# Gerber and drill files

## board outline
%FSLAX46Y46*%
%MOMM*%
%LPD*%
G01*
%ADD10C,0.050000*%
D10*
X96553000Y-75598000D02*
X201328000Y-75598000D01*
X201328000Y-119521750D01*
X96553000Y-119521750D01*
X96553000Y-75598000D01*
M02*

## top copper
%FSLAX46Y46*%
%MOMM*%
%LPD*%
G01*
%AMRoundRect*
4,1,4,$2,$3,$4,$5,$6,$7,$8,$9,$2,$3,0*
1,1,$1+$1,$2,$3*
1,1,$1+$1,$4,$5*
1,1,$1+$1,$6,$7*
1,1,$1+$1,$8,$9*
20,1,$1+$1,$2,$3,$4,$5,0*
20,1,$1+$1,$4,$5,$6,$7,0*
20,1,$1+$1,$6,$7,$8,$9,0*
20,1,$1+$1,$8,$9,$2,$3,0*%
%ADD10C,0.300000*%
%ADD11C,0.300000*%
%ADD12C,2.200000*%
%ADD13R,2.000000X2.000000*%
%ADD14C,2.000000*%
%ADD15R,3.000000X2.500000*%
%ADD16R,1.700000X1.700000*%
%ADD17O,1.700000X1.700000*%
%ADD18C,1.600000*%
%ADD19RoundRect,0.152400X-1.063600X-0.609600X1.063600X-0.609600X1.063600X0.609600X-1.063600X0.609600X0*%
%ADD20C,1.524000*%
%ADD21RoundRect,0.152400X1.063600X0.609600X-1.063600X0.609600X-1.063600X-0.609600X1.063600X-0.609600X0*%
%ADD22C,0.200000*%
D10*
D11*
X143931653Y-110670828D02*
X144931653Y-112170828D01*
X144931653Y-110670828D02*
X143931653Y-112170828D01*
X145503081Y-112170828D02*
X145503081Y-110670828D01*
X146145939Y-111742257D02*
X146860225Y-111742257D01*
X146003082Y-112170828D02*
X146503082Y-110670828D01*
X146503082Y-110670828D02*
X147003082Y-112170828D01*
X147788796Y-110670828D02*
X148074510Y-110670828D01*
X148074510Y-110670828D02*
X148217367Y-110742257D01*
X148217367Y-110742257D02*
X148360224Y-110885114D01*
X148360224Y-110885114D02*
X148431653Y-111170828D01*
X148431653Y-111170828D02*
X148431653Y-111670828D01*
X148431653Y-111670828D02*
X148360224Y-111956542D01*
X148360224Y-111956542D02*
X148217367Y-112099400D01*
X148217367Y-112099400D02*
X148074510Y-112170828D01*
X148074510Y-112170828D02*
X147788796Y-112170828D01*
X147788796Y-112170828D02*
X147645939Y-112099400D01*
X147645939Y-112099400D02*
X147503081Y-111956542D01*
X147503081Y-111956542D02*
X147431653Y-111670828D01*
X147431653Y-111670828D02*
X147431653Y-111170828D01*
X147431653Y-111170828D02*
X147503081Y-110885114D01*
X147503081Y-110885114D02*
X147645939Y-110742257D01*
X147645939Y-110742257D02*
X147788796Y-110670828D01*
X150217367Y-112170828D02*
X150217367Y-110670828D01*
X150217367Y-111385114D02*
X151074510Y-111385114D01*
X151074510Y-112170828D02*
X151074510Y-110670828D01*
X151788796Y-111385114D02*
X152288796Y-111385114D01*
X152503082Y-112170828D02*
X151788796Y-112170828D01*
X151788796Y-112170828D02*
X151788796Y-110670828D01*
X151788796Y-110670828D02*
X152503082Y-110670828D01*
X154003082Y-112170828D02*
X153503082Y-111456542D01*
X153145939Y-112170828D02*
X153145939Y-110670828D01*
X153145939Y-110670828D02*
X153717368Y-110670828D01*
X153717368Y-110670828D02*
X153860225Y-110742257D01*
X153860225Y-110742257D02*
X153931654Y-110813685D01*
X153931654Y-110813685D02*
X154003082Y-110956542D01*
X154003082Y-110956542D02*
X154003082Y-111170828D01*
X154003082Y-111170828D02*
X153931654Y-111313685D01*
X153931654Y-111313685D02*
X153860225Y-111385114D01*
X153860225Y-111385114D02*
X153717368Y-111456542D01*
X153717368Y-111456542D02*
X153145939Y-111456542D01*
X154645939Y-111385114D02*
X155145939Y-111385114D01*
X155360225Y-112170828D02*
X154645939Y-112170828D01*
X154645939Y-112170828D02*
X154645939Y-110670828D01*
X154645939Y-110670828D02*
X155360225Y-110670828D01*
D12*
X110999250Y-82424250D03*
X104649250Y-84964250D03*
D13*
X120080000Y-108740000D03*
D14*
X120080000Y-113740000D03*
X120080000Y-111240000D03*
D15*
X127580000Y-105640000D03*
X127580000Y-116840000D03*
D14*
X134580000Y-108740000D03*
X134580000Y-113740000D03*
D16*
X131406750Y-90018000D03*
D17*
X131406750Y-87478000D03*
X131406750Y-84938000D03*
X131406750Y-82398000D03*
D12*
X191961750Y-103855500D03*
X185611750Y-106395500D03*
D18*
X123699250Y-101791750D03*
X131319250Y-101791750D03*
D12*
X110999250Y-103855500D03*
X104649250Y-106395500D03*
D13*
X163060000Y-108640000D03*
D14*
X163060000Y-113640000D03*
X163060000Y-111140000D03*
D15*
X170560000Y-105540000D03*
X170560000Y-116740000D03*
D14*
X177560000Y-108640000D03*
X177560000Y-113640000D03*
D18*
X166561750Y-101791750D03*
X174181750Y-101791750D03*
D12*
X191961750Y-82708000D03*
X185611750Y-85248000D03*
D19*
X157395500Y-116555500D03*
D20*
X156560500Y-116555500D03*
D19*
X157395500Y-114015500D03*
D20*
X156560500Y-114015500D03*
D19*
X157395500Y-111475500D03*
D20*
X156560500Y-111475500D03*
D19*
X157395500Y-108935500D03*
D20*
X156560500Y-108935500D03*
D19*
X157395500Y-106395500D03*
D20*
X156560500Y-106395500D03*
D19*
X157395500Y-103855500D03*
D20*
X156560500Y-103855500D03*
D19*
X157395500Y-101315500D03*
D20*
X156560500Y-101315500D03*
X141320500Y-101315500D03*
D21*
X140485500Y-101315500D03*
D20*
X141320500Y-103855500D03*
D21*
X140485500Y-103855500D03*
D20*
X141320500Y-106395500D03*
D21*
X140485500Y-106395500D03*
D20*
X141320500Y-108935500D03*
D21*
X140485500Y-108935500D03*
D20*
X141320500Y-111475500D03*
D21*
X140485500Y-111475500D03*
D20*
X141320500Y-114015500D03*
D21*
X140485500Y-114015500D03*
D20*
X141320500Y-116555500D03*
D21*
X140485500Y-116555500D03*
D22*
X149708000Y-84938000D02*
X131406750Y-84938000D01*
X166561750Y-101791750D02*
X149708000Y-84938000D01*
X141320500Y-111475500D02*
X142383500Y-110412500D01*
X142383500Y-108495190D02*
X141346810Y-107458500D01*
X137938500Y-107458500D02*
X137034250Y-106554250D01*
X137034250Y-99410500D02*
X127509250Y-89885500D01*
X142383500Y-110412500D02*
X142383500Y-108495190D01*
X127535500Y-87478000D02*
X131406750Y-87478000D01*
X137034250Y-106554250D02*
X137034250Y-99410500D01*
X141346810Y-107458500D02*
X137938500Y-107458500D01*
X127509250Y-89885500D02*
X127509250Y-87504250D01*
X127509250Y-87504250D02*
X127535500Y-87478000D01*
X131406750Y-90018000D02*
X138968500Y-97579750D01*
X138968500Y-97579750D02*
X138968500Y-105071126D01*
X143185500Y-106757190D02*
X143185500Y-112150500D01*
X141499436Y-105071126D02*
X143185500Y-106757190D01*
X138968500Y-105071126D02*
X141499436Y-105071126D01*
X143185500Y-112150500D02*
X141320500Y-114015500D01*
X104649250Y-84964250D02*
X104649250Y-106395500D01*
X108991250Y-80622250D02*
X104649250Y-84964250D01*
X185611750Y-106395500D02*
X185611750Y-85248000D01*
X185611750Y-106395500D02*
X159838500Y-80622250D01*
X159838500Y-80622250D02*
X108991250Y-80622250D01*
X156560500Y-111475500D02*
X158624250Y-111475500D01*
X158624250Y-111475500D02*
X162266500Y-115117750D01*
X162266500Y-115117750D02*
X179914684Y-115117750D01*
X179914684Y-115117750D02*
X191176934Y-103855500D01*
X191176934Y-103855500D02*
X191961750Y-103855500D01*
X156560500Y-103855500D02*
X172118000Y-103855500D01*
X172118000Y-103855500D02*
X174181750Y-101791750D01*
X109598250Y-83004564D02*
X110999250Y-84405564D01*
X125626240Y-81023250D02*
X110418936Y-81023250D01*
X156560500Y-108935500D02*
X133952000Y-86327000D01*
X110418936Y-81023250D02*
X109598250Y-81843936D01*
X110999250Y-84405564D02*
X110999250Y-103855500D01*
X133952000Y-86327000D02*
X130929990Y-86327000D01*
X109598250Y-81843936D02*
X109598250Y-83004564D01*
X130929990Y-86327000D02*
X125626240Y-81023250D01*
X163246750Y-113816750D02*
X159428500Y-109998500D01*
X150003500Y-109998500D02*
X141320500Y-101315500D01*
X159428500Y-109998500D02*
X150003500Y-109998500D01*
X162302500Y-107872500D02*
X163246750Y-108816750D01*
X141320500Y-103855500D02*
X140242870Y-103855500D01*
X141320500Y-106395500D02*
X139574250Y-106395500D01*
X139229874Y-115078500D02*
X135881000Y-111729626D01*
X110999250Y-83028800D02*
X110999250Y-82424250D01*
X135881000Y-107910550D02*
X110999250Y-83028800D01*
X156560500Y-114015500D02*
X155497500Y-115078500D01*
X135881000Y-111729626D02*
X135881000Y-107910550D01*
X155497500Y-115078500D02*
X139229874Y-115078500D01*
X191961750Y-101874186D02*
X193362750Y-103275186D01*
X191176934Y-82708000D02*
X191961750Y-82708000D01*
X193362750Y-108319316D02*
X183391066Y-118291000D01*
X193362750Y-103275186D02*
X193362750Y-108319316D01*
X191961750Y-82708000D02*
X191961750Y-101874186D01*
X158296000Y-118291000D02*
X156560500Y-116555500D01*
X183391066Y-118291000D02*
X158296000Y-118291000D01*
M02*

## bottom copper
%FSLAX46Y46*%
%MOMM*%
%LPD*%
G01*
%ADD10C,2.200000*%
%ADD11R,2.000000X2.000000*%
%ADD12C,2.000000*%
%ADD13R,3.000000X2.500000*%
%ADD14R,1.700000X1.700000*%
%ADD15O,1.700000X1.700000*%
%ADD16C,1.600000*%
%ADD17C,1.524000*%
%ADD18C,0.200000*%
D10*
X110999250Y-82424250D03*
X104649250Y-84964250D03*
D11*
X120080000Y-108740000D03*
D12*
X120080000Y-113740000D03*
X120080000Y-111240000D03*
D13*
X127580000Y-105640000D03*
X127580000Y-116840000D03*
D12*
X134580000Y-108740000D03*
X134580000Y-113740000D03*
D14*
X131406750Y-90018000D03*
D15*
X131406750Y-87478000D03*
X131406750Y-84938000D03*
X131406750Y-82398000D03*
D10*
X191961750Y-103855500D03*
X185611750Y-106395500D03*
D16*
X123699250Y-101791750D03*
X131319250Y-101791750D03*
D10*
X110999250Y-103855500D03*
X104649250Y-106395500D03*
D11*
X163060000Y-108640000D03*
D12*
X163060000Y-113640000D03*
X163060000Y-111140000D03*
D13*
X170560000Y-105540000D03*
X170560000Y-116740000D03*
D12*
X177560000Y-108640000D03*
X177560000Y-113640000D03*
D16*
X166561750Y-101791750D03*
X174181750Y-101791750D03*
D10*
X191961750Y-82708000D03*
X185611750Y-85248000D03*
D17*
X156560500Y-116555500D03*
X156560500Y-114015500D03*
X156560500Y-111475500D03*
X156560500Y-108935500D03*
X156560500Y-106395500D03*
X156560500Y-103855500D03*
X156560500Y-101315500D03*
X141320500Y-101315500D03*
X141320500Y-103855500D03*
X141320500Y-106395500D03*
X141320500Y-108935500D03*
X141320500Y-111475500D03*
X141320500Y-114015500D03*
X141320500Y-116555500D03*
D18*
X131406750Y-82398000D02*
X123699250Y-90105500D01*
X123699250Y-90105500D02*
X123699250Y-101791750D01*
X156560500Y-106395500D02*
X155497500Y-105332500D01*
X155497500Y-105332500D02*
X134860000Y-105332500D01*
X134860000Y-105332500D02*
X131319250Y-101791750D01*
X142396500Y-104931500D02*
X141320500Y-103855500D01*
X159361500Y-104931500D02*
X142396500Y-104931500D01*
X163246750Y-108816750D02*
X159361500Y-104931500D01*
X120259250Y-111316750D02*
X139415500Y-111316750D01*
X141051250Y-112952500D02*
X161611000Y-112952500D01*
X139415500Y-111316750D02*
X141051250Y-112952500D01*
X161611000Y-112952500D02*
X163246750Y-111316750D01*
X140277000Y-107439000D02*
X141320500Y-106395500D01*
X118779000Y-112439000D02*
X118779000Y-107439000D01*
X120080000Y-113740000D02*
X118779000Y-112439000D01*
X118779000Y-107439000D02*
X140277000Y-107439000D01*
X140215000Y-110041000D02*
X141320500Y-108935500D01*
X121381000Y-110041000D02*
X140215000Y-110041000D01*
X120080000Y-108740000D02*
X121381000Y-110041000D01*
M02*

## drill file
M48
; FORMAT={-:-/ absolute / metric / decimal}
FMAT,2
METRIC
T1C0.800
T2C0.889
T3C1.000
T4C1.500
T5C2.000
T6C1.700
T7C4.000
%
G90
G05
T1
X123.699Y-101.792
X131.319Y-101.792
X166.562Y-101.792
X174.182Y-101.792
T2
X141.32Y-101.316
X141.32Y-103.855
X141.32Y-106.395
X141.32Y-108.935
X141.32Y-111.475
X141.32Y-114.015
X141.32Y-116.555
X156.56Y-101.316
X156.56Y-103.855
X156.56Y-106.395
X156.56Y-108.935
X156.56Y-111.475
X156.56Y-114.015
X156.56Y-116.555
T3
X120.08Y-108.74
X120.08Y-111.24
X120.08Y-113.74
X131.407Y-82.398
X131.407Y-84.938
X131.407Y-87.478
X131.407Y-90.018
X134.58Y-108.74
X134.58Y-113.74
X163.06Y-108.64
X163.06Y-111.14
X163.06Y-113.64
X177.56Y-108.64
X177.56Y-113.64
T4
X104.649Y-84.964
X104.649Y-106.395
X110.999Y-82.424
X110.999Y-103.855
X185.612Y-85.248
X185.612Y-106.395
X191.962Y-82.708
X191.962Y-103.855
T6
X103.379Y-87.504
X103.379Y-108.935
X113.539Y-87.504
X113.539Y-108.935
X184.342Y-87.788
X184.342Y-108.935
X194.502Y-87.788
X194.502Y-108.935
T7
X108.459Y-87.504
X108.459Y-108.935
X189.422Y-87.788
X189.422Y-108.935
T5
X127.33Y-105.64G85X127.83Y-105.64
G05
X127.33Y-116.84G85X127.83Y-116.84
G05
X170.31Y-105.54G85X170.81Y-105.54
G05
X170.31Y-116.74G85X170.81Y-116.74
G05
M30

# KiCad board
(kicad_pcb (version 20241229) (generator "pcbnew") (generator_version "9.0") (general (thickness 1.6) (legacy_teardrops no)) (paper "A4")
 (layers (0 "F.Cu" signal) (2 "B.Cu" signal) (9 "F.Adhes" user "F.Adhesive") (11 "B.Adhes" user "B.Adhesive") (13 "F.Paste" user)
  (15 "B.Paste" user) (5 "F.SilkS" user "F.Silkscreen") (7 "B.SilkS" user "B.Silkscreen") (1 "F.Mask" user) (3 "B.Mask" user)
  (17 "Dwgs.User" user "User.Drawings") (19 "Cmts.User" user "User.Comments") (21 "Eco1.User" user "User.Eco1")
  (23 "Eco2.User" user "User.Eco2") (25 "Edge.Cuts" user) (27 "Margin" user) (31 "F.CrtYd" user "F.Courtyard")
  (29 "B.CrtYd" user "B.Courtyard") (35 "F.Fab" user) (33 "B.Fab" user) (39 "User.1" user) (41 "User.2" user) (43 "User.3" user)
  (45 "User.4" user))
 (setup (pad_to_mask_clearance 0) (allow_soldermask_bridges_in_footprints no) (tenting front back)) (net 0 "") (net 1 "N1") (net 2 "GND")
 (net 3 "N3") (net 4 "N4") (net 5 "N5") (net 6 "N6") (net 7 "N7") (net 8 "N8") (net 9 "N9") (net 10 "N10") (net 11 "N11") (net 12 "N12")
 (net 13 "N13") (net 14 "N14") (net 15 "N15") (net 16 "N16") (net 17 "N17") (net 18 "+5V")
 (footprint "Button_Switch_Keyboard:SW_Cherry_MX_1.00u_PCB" (layer "F.Cu") (at 110.99925 82.42425)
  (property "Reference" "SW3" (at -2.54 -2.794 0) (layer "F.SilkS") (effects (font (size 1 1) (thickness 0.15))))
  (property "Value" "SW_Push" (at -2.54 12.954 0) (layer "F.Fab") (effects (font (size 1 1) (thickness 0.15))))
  (pad "" np_thru_hole circle (at -7.62 5.08) (size 1.7 1.7) (drill 1.7) (layers "*.Cu" "*.Mask"))
  (pad "" np_thru_hole circle (at -2.54 5.08) (size 4 4) (drill 4) (layers "*.Cu" "*.Mask"))
  (pad "" np_thru_hole circle (at 2.54 5.08) (size 1.7 1.7) (drill 1.7) (layers "*.Cu" "*.Mask"))
  (pad "1" thru_hole circle (at 0 0) (size 2.2 2.2) (drill 1.5) (layers "*.Cu" "*.Mask") (remove_unused_layers no) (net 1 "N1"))
  (pad "2" thru_hole circle (at -6.35 2.54) (size 2.2 2.2) (drill 1.5) (layers "*.Cu" "*.Mask") (remove_unused_layers no) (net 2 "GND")))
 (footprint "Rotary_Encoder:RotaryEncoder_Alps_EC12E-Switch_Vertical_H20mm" (layer "F.Cu") (at 120.08 108.74)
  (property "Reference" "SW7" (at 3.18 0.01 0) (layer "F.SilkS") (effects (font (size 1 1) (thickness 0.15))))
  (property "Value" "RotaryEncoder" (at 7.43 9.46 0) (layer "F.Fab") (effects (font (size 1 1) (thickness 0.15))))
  (pad "A" thru_hole rect (at 0 0) (size 2 2) (drill 1) (layers "*.Cu" "*.Mask") (remove_unused_layers no) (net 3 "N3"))
  (pad "B" thru_hole circle (at 0 5) (size 2 2) (drill 1) (layers "*.Cu" "*.Mask") (remove_unused_layers no) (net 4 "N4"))
  (pad "C" thru_hole circle (at 0 2.5) (size 2 2) (drill 1) (layers "*.Cu" "*.Mask") (remove_unused_layers no) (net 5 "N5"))
  (pad "MP" thru_hole rect (at 7.5 -3.1) (size 3 2.5) (drill oval 2.5 2) (layers "*.Cu" "*.Mask") (remove_unused_layers no))
  (pad "MP" thru_hole rect (at 7.5 8.1) (size 3 2.5) (drill oval 2.5 2) (layers "*.Cu" "*.Mask") (remove_unused_layers no))
  (pad "S1" thru_hole circle (at 14.5 0) (size 2 2) (drill 1) (layers "*.Cu" "*.Mask") (remove_unused_layers no))
  (pad "S2" thru_hole circle (at 14.5 5) (size 2 2) (drill 1) (layers "*.Cu" "*.Mask") (remove_unused_layers no)))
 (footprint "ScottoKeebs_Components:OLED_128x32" (layer "F.Cu") (at 129.80675 80.218)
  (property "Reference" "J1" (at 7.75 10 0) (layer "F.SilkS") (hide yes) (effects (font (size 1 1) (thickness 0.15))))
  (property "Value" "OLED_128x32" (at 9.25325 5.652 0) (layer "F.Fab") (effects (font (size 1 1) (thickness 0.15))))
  (pad "1" thru_hole rect (at 1.6 9.8 180) (size 1.7 1.7) (drill 1) (layers "*.Cu" "*.Mask") (remove_unused_layers no) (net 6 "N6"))
  (pad "2" thru_hole oval (at 1.6 7.26 180) (size 1.7 1.7) (drill 1) (layers "*.Cu" "*.Mask") (remove_unused_layers no) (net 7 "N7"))
  (pad "3" thru_hole oval (at 1.6 4.72 180) (size 1.7 1.7) (drill 1) (layers "*.Cu" "*.Mask") (remove_unused_layers no) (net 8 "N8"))
  (pad "4" thru_hole oval (at 1.6 2.18 180) (size 1.7 1.7) (drill 1) (layers "*.Cu" "*.Mask") (remove_unused_layers no) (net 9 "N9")))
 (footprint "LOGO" (layer "F.Cu") (at 148.86 95.36)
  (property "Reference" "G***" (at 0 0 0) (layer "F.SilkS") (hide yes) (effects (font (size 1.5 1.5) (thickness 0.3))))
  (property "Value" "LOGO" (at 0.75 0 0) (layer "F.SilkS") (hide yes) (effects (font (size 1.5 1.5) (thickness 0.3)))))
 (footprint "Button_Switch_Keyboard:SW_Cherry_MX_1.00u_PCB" (layer "F.Cu") (at 191.96175 103.8555)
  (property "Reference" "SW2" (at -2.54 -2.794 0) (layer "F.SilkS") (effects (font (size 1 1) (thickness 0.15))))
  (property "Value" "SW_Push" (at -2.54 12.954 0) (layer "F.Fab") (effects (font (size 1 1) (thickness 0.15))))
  (pad "" np_thru_hole circle (at -7.62 5.08) (size 1.7 1.7) (drill 1.7) (layers "*.Cu" "*.Mask"))
  (pad "" np_thru_hole circle (at -2.54 5.08) (size 4 4) (drill 4) (layers "*.Cu" "*.Mask"))
  (pad "" np_thru_hole circle (at 2.54 5.08) (size 1.7 1.7) (drill 1.7) (layers "*.Cu" "*.Mask"))
  (pad "1" thru_hole circle (at 0 0) (size 2.2 2.2) (drill 1.5) (layers "*.Cu" "*.Mask") (remove_unused_layers no) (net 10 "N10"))
  (pad "2" thru_hole circle (at -6.35 2.54) (size 2.2 2.2) (drill 1.5) (layers "*.Cu" "*.Mask") (remove_unused_layers no) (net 2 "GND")))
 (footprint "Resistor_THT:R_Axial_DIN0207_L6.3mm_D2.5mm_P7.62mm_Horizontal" (layer "F.Cu") (at 123.69925 101.79175)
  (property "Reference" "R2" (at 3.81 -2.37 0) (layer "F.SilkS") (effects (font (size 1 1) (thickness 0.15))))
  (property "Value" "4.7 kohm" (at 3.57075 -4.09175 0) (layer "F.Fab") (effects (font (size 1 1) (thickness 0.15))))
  (pad "1" thru_hole circle (at 0 0) (size 1.6 1.6) (drill 0.8) (layers "*.Cu" "*.Mask") (remove_unused_layers no) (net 9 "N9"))
  (pad "2" thru_hole circle (at 7.62 0) (size 1.6 1.6) (drill 0.8) (layers "*.Cu" "*.Mask") (remove_unused_layers no) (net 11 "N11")))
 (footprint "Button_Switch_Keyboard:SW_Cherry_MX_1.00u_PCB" (layer "F.Cu") (at 110.99925 103.8555)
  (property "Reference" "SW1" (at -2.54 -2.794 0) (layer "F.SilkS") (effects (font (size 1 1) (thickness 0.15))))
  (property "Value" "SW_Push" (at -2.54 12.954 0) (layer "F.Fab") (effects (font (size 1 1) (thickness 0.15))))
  (pad "" np_thru_hole circle (at -7.62 5.08) (size 1.7 1.7) (drill 1.7) (layers "*.Cu" "*.Mask"))
  (pad "" np_thru_hole circle (at -2.54 5.08) (size 4 4) (drill 4) (layers "*.Cu" "*.Mask"))
  (pad "" np_thru_hole circle (at 2.54 5.08) (size 1.7 1.7) (drill 1.7) (layers "*.Cu" "*.Mask"))
  (pad "1" thru_hole circle (at 0 0) (size 2.2 2.2) (drill 1.5) (layers "*.Cu" "*.Mask") (remove_unused_layers no) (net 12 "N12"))
  (pad "2" thru_hole circle (at -6.35 2.54) (size 2.2 2.2) (drill 1.5) (layers "*.Cu" "*.Mask") (remove_unused_layers no) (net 2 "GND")))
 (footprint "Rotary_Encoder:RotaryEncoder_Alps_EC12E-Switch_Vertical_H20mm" (layer "F.Cu") (at 163.06 108.64)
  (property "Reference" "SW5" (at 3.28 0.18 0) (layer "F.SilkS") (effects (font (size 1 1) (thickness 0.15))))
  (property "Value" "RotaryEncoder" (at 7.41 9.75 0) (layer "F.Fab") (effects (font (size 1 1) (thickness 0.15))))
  (pad "A" thru_hole rect (at 0 0) (size 2 2) (drill 1) (layers "*.Cu" "*.Mask") (remove_unused_layers no) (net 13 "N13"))
  (pad "B" thru_hole circle (at 0 5) (size 2 2) (drill 1) (layers "*.Cu" "*.Mask") (remove_unused_layers no) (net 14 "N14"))
  (pad "C" thru_hole circle (at 0 2.5) (size 2 2) (drill 1) (layers "*.Cu" "*.Mask") (remove_unused_layers no) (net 5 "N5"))
  (pad "MP" thru_hole rect (at 7.5 -3.1) (size 3 2.5) (drill oval 2.5 2) (layers "*.Cu" "*.Mask") (remove_unused_layers no))
  (pad "MP" thru_hole rect (at 7.5 8.1) (size 3 2.5) (drill oval 2.5 2) (layers "*.Cu" "*.Mask") (remove_unused_layers no))
  (pad "S1" thru_hole circle (at 14.5 0) (size 2 2) (drill 1) (layers "*.Cu" "*.Mask") (remove_unused_layers no))
  (pad "S2" thru_hole circle (at 14.5 5) (size 2 2) (drill 1) (layers "*.Cu" "*.Mask") (remove_unused_layers no)))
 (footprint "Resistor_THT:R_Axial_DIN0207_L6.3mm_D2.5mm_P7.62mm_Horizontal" (layer "F.Cu") (at 166.56175 101.79175)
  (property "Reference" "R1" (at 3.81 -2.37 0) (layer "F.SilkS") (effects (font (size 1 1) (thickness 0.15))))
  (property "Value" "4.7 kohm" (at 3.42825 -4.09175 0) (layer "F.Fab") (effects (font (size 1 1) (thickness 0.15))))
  (pad "1" thru_hole circle (at 0 0) (size 1.6 1.6) (drill 0.8) (layers "*.Cu" "*.Mask") (remove_unused_layers no) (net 8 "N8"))
  (pad "2" thru_hole circle (at 7.62 0) (size 1.6 1.6) (drill 0.8) (layers "*.Cu" "*.Mask") (remove_unused_layers no) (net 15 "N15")))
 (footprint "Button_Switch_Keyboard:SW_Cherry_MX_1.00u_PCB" (layer "F.Cu") (at 191.96175 82.708)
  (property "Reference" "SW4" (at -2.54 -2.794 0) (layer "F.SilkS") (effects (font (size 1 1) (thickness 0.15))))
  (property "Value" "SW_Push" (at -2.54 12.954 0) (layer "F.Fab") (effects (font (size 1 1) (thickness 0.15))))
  (pad "" np_thru_hole circle (at -7.62 5.08) (size 1.7 1.7) (drill 1.7) (layers "*.Cu" "*.Mask"))
  (pad "" np_thru_hole circle (at -2.54 5.08) (size 4 4) (drill 4) (layers "*.Cu" "*.Mask"))
  (pad "" np_thru_hole circle (at 2.54 5.08) (size 1.7 1.7) (drill 1.7) (layers "*.Cu" "*.Mask"))
  (pad "1" thru_hole circle (at 0 0) (size 2.2 2.2) (drill 1.5) (layers "*.Cu" "*.Mask") (remove_unused_layers no) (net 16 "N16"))
  (pad "2" thru_hole circle (at -6.35 2.54) (size 2.2 2.2) (drill 1.5) (layers "*.Cu" "*.Mask") (remove_unused_layers no) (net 2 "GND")))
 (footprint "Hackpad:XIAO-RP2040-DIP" (layer "F.Cu") (at 148.9405 108.9355 180)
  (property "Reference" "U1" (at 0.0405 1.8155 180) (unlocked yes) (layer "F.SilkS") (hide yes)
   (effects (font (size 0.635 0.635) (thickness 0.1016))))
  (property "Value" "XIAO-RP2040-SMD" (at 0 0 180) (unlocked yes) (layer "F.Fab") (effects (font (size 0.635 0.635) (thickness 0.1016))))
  (pad "1" smd roundrect (at -8.455 -7.62) (size 2.432 1.524) (layers "F.Cu" "F.Mask") (roundrect_rratio 0.1) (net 16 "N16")
   (thermal_bridge_angle 45))
  (pad "1" thru_hole circle (at -7.62 -7.62) (size 1.524 1.524) (drill 0.889) (layers "*.Cu" "*.Mask") (remove_unused_layers no)
   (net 16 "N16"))
  (pad "2" smd roundrect (at -8.455 -5.08) (size 2.432 1.524) (layers "F.Cu" "F.Mask") (roundrect_rratio 0.1) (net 1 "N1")
   (thermal_bridge_angle 45))
  (pad "2" thru_hole circle (at -7.62 -5.08) (size 1.524 1.524) (drill 0.889) (layers "*.Cu" "*.Mask") (remove_unused_layers no)
   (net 1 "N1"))
  (pad "3" smd roundrect (at -8.455 -2.54) (size 2.432 1.524) (layers "F.Cu" "F.Mask") (roundrect_rratio 0.1) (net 10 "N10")
   (thermal_bridge_angle 45))
  (pad "3" thru_hole circle (at -7.62 -2.54) (size 1.524 1.524) (drill 0.889) (layers "*.Cu" "*.Mask") (remove_unused_layers no)
   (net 10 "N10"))
  (pad "4" smd roundrect (at -8.455 0) (size 2.432 1.524) (layers "F.Cu" "F.Mask") (roundrect_rratio 0.1) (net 12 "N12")
   (thermal_bridge_angle 45))
  (pad "4" thru_hole circle (at -7.62 0) (size 1.524 1.524) (drill 0.889) (layers "*.Cu" "*.Mask") (remove_unused_layers no) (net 12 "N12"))
  (pad "5" smd roundrect (at -8.455 2.54) (size 2.432 1.524) (layers "F.Cu" "F.Mask") (roundrect_rratio 0.1) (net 11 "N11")
   (thermal_bridge_angle 45))
  (pad "5" thru_hole circle (at -7.62 2.54) (size 1.524 1.524) (drill 0.889) (layers "*.Cu" "*.Mask") (remove_unused_layers no)
   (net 11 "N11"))
  (pad "6" smd roundrect (at -8.455 5.08) (size 2.432 1.524) (layers "F.Cu" "F.Mask") (roundrect_rratio 0.1) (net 15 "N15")
   (thermal_bridge_angle 45))
  (pad "6" thru_hole circle (at -7.62 5.08) (size 1.524 1.524) (drill 0.889) (layers "*.Cu" "*.Mask") (remove_unused_layers no)
   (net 15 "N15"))
  (pad "7" smd roundrect (at -8.455 7.62) (size 2.432 1.524) (layers "F.Cu" "F.Mask") (roundrect_rratio 0.1) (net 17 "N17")
   (thermal_bridge_angle 45))
  (pad "7" thru_hole circle (at -7.62 7.62) (size 1.524 1.524) (drill 0.889) (layers "*.Cu" "*.Mask") (remove_unused_layers no)
   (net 17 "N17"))
  (pad "8" thru_hole circle (at 7.62 7.62 180) (size 1.524 1.524) (drill 0.889) (layers "*.Cu" "*.Mask") (remove_unused_layers no)
   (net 14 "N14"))
  (pad "8" smd roundrect (at 8.455 7.62 180) (size 2.432 1.524) (layers "F.Cu" "F.Mask") (roundrect_rratio 0.1) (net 14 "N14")
   (thermal_bridge_angle 45))
  (pad "9" thru_hole circle (at 7.62 5.08 180) (size 1.524 1.524) (drill 0.889) (layers "*.Cu" "*.Mask") (remove_unused_layers no)
   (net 13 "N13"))
  (pad "9" smd roundrect (at 8.455 5.08 180) (size 2.432 1.524) (layers "F.Cu" "F.Mask") (roundrect_rratio 0.1) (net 13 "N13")
   (thermal_bridge_angle 45))
  (pad "10" thru_hole circle (at 7.62 2.54 180) (size 1.524 1.524) (drill 0.889) (layers "*.Cu" "*.Mask") (remove_unused_layers no)
   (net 4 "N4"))
  (pad "10" smd roundrect (at 8.455 2.54 180) (size 2.432 1.524) (layers "F.Cu" "F.Mask") (roundrect_rratio 0.1) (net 4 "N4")
   (thermal_bridge_angle 45))
  (pad "11" thru_hole circle (at 7.62 0 180) (size 1.524 1.524) (drill 0.889) (layers "*.Cu" "*.Mask") (remove_unused_layers no)
   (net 3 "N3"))
  (pad "11" smd roundrect (at 8.455 0 180) (size 2.432 1.524) (layers "F.Cu" "F.Mask") (roundrect_rratio 0.1) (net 3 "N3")
   (thermal_bridge_angle 45))
  (pad "12" thru_hole circle (at 7.62 -2.54 180) (size 1.524 1.524) (drill 0.889) (layers "*.Cu" "*.Mask") (remove_unused_layers no)
   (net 7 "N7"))
  (pad "12" smd roundrect (at 8.455 -2.54 180) (size 2.432 1.524) (layers "F.Cu" "F.Mask") (roundrect_rratio 0.1) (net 7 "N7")
   (thermal_bridge_angle 45))
  (pad "13" thru_hole circle (at 7.62 -5.08 180) (size 1.524 1.524) (drill 0.889) (layers "*.Cu" "*.Mask") (remove_unused_layers no)
   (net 6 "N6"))
  (pad "13" smd roundrect (at 8.455 -5.08 180) (size 2.432 1.524) (layers "F.Cu" "F.Mask") (roundrect_rratio 0.1) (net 6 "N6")
   (thermal_bridge_angle 45))
  (pad "14" thru_hole circle (at 7.62 -7.62 180) (size 1.524 1.524) (drill 0.889) (layers "*.Cu" "*.Mask") (remove_unused_layers no)
   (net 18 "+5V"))
  (pad "14" smd roundrect (at 8.455 -7.62 180) (size 2.432 1.524) (layers "F.Cu" "F.Mask") (roundrect_rratio 0.1) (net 18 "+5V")
   (thermal_bridge_angle 45)))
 (gr_rect (start 96.553 75.598) (end 201.328 119.52175) (stroke (width 0.05) (type default)) (fill no) (layer "Edge.Cuts"))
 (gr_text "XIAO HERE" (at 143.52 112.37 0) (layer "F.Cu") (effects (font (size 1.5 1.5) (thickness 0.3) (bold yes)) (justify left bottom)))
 (segment (start 131.40675 82.398) (end 123.69925 90.1055) (width 0.2) (layer "B.Cu") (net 9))
 (segment (start 123.69925 90.1055) (end 123.69925 101.79175) (width 0.2) (layer "B.Cu") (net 9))
 (segment (start 149.708 84.938) (end 131.40675 84.938) (width 0.2) (layer "F.Cu") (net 8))
 (segment (start 166.56175 101.79175) (end 149.708 84.938) (width 0.2) (layer "F.Cu") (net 8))
 (segment (start 141.3205 111.4755) (end 142.3835 110.4125) (width 0.2) (layer "F.Cu") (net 7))
 (segment (start 142.3835 108.49519) (end 141.34681 107.4585) (width 0.2) (layer "F.Cu") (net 7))
 (segment (start 137.9385 107.4585) (end 137.03425 106.55425) (width 0.2) (layer "F.Cu") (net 7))
 (segment (start 137.03425 99.4105) (end 127.50925 89.8855) (width 0.2) (layer "F.Cu") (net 7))
 (segment (start 142.3835 110.4125) (end 142.3835 108.49519) (width 0.2) (layer "F.Cu") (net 7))
 (segment (start 127.5355 87.478) (end 131.40675 87.478) (width 0.2) (layer "F.Cu") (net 7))
 (segment (start 137.03425 106.55425) (end 137.03425 99.4105) (width 0.2) (layer "F.Cu") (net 7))
 (segment (start 141.34681 107.4585) (end 137.9385 107.4585) (width 0.2) (layer "F.Cu") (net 7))
 (segment (start 127.50925 89.8855) (end 127.50925 87.50425) (width 0.2) (layer "F.Cu") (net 7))
 (segment (start 127.50925 87.50425) (end 127.5355 87.478) (width 0.2) (layer "F.Cu") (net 7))
 (segment (start 131.40675 90.018) (end 138.9685 97.57975) (width 0.2) (layer "F.Cu") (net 6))
 (segment (start 138.9685 97.57975) (end 138.9685 105.071126) (width 0.2) (layer "F.Cu") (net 6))
 (segment (start 143.1855 106.75719) (end 143.1855 112.1505) (width 0.2) (layer "F.Cu") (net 6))
 (segment (start 141.499436 105.071126) (end 143.1855 106.75719) (width 0.2) (layer "F.Cu") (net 6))
 (segment (start 138.9685 105.071126) (end 141.499436 105.071126) (width 0.2) (layer "F.Cu") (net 6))
 (segment (start 143.1855 112.1505) (end 141.3205 114.0155) (width 0.2) (layer "F.Cu") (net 6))
 (segment (start 104.64925 84.96425) (end 104.64925 106.3955) (width 0.2) (layer "F.Cu") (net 2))
 (segment (start 108.99125 80.62225) (end 104.64925 84.96425) (width 0.2) (layer "F.Cu") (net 2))
 (segment (start 185.61175 106.3955) (end 185.61175 85.248) (width 0.2) (layer "F.Cu") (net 2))
 (segment (start 185.61175 106.3955) (end 159.8385 80.62225) (width 0.2) (layer "F.Cu") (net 2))
 (segment (start 159.8385 80.62225) (end 108.99125 80.62225) (width 0.2) (layer "F.Cu") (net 2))
 (segment (start 156.5605 111.4755) (end 158.62425 111.4755) (width 0.2) (layer "F.Cu") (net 10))
 (segment (start 158.62425 111.4755) (end 162.2665 115.11775) (width 0.2) (layer "F.Cu") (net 10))
 (segment (start 162.2665 115.11775) (end 179.914684 115.11775) (width 0.2) (layer "F.Cu") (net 10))
 (segment (start 179.914684 115.11775) (end 191.176934 103.8555) (width 0.2) (layer "F.Cu") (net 10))
 (segment (start 191.176934 103.8555) (end 191.96175 103.8555) (width 0.2) (layer "F.Cu") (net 10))
 (segment (start 156.5605 103.8555) (end 172.118 103.8555) (width 0.2) (layer "F.Cu") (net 15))
 (segment (start 172.118 103.8555) (end 174.18175 101.79175) (width 0.2) (layer "F.Cu") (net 15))
 (segment (start 156.5605 106.3955) (end 155.4975 105.3325) (width 0.2) (layer "B.Cu") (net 11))
 (segment (start 155.4975 105.3325) (end 134.86 105.3325) (width 0.2) (layer "B.Cu") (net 11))
 (segment (start 134.86 105.3325) (end 131.31925 101.79175) (width 0.2) (layer "B.Cu") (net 11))
 (segment (start 109.59825 83.004564) (end 110.99925 84.405564) (width 0.2) (layer "F.Cu") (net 12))
 (segment (start 125.62624 81.02325) (end 110.418936 81.02325) (width 0.2) (layer "F.Cu") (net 12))
 (segment (start 156.5605 108.9355) (end 133.952 86.327) (width 0.2) (layer "F.Cu") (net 12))
 (segment (start 110.418936 81.02325) (end 109.59825 81.843936) (width 0.2) (layer "F.Cu") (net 12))
 (segment (start 110.99925 84.405564) (end 110.99925 103.8555) (width 0.2) (layer "F.Cu") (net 12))
 (segment (start 133.952 86.327) (end 130.92999 86.327) (width 0.2) (layer "F.Cu") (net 12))
 (segment (start 109.59825 81.843936) (end 109.59825 83.004564) (width 0.2) (layer "F.Cu") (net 12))
 (segment (start 130.92999 86.327) (end 125.62624 81.02325) (width 0.2) (layer "F.Cu") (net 12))
 (segment (start 163.24675 113.81675) (end 159.4285 109.9985) (width 0.2) (layer "F.Cu") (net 14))
 (segment (start 150.0035 109.9985) (end 141.3205 101.3155) (width 0.2) (layer "F.Cu") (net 14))
 (segment (start 159.4285 109.9985) (end 150.0035 109.9985) (width 0.2) (layer "F.Cu") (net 14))
 (segment (start 162.3025 107.8725) (end 163.24675 108.81675) (width 0.2) (layer "F.Cu") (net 13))
 (segment (start 141.3205 103.8555) (end 140.24287 103.8555) (width 0.2) (layer "F.Cu") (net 13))
 (segment (start 142.3965 104.9315) (end 141.3205 103.8555) (width 0.2) (layer "B.Cu") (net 13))
 (segment (start 159.3615 104.9315) (end 142.3965 104.9315) (width 0.2) (layer "B.Cu") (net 13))
 (segment (start 163.24675 108.81675) (end 159.3615 104.9315) (width 0.2) (layer "B.Cu") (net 13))
 (segment (start 120.25925 111.31675) (end 139.4155 111.31675) (width 0.2) (layer "B.Cu") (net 5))
 (segment (start 141.05125 112.9525) (end 161.611 112.9525) (width 0.2) (layer "B.Cu") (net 5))
 (segment (start 139.4155 111.31675) (end 141.05125 112.9525) (width 0.2) (layer "B.Cu") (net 5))
 (segment (start 161.611 112.9525) (end 163.24675 111.31675) (width 0.2) (layer "B.Cu") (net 5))
 (segment (start 141.3205 106.3955) (end 139.57425 106.3955) (width 0.2) (layer "F.Cu") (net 4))
 (segment (start 140.277 107.439) (end 141.3205 106.3955) (width 0.2) (layer "B.Cu") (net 4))
 (segment (start 118.779 112.439) (end 118.779 107.439) (width 0.2) (layer "B.Cu") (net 4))
 (segment (start 120.08 113.74) (end 118.779 112.439) (width 0.2) (layer "B.Cu") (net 4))
 (segment (start 118.779 107.439) (end 140.277 107.439) (width 0.2) (layer "B.Cu") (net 4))
 (segment (start 140.215 110.041) (end 141.3205 108.9355) (width 0.2) (layer "B.Cu") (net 3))
 (segment (start 121.381 110.041) (end 140.215 110.041) (width 0.2) (layer "B.Cu") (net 3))
 (segment (start 120.08 108.74) (end 121.381 110.041) (width 0.2) (layer "B.Cu") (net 3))
 (segment (start 139.229874 115.0785) (end 135.881 111.729626) (width 0.2) (layer "F.Cu") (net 1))
 (segment (start 110.99925 83.0288) (end 110.99925 82.42425) (width 0.2) (layer "F.Cu") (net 1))
 (segment (start 135.881 107.91055) (end 110.99925 83.0288) (width 0.2) (layer "F.Cu") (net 1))
 (segment (start 156.5605 114.0155) (end 155.4975 115.0785) (width 0.2) (layer "F.Cu") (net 1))
 (segment (start 135.881 111.729626) (end 135.881 107.91055) (width 0.2) (layer "F.Cu") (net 1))
 (segment (start 155.4975 115.0785) (end 139.229874 115.0785) (width 0.2) (layer "F.Cu") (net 1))
 (segment (start 191.96175 101.874186) (end 193.36275 103.275186) (width 0.2) (layer "F.Cu") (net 16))
 (segment (start 191.176934 82.708) (end 191.96175 82.708) (width 0.2) (layer "F.Cu") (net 16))
 (segment (start 193.36275 108.319316) (end 183.391066 118.291) (width 0.2) (layer "F.Cu") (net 16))
 (segment (start 193.36275 103.275186) (end 193.36275 108.319316) (width 0.2) (layer "F.Cu") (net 16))
 (segment (start 191.96175 82.708) (end 191.96175 101.874186) (width 0.2) (layer "F.Cu") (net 16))
 (segment (start 158.296 118.291) (end 156.5605 116.5555) (width 0.2) (layer "F.Cu") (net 16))
 (segment (start 183.391066 118.291) (end 158.296 118.291) (width 0.2) (layer "F.Cu") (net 16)))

